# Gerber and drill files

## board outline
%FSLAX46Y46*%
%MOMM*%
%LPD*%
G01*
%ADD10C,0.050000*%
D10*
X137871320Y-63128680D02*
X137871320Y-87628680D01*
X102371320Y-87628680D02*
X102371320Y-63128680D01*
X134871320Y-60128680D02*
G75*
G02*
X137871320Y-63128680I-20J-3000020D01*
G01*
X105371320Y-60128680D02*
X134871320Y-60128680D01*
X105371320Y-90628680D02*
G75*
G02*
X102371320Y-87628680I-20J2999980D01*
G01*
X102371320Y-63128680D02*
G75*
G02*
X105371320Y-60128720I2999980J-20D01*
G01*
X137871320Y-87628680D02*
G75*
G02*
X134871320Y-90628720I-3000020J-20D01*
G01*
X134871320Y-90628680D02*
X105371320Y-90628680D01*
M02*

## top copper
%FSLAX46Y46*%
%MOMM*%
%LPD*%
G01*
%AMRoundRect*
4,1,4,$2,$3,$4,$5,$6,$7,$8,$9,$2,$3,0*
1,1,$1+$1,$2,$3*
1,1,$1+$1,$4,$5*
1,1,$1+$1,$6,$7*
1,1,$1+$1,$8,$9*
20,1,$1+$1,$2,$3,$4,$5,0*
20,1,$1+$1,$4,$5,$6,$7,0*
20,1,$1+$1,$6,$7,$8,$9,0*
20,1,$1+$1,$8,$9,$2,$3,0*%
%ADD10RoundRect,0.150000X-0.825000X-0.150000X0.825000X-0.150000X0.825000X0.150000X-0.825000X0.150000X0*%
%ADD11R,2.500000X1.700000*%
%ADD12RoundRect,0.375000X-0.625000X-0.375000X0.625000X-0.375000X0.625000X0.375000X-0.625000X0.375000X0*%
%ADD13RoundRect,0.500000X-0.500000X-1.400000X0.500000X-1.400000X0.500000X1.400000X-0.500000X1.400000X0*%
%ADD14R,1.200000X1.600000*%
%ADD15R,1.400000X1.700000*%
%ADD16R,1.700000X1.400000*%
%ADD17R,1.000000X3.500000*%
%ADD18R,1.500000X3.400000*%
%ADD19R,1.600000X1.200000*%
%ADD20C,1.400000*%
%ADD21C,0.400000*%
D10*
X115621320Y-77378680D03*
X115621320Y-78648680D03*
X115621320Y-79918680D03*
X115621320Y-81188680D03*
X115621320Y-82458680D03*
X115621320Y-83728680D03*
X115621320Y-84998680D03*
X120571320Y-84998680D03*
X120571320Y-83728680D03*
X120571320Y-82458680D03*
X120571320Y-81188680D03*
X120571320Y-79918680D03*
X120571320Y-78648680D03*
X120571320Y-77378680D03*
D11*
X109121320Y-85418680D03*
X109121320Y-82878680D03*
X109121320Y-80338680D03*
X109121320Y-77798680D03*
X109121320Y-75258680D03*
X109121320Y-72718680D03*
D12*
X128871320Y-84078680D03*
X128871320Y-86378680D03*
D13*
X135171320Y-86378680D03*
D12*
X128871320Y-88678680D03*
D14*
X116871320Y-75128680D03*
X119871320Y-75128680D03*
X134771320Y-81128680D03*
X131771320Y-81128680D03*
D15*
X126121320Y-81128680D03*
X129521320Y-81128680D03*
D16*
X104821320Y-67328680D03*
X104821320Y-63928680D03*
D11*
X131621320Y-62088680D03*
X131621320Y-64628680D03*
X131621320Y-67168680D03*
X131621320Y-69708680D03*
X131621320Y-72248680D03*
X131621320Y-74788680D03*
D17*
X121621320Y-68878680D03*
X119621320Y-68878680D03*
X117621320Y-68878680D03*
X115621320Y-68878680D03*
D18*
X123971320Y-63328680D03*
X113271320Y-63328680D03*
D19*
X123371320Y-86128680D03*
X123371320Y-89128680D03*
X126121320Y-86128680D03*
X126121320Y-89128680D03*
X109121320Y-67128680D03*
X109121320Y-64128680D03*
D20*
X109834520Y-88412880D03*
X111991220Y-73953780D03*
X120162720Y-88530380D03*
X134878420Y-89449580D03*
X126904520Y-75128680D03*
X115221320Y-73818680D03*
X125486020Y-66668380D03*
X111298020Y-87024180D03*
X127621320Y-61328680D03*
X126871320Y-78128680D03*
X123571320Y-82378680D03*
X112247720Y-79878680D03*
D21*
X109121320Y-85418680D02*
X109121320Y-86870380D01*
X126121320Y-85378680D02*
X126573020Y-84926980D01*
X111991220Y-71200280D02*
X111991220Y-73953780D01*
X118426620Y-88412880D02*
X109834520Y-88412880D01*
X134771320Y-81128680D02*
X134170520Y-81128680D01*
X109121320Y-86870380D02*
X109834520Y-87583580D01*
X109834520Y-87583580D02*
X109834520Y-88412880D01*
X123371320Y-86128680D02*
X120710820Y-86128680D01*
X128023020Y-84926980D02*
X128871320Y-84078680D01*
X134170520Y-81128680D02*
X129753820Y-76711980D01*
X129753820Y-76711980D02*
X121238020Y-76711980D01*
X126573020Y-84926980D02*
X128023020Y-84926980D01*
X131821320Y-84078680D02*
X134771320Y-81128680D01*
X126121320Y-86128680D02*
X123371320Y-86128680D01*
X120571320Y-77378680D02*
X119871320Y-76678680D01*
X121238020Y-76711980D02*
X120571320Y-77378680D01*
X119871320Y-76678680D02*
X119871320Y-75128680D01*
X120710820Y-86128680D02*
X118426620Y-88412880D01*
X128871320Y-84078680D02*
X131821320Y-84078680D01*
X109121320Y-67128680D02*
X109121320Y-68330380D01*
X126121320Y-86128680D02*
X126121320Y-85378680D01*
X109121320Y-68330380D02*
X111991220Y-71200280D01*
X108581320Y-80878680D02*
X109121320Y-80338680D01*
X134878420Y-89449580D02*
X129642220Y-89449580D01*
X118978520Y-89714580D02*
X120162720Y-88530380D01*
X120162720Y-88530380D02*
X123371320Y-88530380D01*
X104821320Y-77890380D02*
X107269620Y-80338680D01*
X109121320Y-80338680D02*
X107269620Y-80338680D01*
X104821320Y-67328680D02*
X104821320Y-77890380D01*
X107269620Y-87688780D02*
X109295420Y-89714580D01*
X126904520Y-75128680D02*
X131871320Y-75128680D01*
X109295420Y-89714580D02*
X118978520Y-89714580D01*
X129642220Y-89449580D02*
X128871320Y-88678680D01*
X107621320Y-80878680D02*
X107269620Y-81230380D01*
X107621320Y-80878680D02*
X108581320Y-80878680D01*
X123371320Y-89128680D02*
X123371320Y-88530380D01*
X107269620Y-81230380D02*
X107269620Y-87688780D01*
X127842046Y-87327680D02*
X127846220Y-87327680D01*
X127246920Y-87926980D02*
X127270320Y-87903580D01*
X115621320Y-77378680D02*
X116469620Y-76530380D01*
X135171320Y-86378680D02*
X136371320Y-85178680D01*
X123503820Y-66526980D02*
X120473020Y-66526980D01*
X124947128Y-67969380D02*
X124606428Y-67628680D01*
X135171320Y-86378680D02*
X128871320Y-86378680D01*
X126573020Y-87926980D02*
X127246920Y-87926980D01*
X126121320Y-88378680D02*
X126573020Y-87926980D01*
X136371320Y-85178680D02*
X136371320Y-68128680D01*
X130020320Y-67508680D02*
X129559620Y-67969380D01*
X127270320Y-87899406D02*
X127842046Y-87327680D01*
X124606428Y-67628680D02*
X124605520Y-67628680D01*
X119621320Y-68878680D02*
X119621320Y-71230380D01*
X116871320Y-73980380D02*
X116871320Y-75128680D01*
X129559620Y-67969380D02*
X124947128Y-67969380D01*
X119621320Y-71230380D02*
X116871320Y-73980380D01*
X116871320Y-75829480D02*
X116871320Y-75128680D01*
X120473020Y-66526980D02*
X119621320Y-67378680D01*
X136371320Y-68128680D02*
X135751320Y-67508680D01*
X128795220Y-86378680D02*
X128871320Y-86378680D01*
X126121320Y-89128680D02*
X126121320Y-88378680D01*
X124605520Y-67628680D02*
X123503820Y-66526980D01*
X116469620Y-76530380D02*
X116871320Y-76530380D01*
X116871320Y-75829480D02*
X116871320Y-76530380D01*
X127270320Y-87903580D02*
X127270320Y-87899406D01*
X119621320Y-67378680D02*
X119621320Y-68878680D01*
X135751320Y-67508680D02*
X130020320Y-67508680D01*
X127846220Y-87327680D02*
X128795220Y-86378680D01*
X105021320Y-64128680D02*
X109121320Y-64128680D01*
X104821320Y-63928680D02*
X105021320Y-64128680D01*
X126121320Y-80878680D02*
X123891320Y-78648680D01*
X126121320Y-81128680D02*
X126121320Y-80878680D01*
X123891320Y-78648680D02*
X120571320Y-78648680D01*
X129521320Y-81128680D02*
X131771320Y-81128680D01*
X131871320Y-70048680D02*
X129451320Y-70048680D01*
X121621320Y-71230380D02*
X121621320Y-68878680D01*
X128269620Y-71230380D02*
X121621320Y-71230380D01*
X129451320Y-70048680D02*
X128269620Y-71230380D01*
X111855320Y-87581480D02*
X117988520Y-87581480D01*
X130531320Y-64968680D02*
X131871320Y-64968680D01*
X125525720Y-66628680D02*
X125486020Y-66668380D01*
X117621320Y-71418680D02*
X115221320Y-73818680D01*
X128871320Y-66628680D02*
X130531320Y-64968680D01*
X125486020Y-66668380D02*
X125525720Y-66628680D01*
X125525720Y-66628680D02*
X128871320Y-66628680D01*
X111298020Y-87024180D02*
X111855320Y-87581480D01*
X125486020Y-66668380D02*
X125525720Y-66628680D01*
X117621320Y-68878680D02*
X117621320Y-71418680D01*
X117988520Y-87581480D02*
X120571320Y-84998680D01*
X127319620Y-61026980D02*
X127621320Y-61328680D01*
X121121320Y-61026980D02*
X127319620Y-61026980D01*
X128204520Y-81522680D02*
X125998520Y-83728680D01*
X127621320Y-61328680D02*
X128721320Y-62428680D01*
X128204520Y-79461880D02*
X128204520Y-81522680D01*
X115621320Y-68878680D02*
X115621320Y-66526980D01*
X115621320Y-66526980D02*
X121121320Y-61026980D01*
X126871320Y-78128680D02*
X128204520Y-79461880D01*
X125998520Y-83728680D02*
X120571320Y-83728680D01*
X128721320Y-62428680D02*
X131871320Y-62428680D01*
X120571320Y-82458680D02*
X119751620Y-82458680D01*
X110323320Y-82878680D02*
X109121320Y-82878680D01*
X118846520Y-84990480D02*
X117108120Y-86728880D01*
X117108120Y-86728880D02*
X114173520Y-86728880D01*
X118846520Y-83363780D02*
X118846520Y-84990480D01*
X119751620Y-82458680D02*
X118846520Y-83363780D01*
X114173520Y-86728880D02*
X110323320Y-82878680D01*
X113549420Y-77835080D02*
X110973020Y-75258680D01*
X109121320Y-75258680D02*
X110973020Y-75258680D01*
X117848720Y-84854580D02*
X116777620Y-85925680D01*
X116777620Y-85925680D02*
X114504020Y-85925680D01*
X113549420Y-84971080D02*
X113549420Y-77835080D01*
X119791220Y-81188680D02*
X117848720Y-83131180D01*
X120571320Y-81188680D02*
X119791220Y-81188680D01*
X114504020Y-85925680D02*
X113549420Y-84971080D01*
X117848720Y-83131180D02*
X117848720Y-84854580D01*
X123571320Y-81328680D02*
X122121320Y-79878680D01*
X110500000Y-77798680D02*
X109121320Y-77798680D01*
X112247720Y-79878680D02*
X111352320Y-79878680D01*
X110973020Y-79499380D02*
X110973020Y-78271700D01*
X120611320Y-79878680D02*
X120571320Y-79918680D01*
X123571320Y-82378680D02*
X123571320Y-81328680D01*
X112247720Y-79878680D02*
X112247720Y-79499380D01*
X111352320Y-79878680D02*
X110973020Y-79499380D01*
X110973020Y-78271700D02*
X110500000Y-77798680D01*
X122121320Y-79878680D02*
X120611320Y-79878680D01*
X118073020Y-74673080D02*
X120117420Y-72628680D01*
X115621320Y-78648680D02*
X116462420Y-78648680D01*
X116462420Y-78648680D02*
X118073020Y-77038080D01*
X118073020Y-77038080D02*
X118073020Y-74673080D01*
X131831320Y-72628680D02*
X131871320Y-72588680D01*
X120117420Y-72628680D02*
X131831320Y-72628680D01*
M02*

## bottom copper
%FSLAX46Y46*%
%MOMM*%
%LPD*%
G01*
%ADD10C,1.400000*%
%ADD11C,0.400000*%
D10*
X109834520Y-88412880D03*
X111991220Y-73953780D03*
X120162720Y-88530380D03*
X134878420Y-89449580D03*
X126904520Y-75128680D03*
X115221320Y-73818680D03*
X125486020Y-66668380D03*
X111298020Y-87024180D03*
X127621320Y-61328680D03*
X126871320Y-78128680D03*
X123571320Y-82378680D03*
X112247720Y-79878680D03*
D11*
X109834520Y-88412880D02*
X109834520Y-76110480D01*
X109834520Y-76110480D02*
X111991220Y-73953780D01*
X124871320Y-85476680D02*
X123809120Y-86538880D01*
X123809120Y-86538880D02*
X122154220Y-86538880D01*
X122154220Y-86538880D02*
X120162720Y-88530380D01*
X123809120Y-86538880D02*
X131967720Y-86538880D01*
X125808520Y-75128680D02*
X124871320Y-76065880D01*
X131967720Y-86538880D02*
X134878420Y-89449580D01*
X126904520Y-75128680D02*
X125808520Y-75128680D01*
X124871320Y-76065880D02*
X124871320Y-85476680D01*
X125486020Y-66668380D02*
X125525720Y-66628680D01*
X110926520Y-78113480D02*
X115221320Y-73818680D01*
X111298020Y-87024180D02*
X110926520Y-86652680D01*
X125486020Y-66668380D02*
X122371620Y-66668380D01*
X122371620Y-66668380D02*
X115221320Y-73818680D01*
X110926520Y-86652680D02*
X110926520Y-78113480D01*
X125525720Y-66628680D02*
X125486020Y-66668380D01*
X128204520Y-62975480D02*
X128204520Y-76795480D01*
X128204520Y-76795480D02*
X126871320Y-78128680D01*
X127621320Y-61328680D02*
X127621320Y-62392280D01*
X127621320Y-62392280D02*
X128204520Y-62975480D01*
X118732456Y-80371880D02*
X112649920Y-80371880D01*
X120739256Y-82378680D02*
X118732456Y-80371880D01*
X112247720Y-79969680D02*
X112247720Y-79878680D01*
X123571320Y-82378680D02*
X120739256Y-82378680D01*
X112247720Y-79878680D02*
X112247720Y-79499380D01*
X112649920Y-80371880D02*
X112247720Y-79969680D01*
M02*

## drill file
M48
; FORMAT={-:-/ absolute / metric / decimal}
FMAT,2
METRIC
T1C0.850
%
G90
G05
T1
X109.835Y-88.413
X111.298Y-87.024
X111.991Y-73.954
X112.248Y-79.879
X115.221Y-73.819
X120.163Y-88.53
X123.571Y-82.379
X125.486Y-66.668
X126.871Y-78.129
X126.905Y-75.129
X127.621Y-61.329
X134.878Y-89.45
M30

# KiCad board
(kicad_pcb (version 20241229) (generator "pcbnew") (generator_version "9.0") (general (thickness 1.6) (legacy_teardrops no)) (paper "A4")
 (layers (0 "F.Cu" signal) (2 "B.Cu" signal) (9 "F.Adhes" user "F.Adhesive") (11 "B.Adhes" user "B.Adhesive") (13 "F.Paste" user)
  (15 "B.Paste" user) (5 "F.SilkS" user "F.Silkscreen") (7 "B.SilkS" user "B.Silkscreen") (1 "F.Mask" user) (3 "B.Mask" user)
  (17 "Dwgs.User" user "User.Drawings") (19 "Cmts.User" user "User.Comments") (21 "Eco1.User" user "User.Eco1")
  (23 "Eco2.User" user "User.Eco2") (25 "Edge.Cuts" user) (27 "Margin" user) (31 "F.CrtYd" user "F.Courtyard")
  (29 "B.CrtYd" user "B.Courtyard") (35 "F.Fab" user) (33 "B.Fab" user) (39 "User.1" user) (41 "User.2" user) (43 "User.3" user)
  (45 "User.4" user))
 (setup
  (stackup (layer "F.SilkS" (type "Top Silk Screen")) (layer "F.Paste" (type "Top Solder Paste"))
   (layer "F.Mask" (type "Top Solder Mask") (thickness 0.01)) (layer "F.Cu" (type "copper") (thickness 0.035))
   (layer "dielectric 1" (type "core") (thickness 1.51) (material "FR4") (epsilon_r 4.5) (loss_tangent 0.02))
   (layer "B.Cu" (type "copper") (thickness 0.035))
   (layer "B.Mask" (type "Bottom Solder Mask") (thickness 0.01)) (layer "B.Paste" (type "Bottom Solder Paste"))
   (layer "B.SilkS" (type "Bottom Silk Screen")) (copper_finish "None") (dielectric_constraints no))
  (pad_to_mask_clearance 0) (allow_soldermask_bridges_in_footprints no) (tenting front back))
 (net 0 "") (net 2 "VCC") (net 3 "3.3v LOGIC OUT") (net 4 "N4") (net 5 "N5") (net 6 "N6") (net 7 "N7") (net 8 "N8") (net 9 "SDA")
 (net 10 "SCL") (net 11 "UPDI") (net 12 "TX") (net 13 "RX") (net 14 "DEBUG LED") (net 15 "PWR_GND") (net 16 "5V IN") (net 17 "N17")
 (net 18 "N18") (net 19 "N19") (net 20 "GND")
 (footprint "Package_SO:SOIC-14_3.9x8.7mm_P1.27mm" (layer "F.Cu") (at 118.09632 81.18868)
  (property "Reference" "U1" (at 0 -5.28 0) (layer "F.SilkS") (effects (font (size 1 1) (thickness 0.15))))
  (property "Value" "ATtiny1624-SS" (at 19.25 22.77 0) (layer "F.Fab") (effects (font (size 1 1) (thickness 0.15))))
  (pad "1" smd roundrect (at -2.475 -3.81) (size 1.95 0.6) (layers "F.Cu" "F.Mask" "F.Paste") (roundrect_rratio 0.25) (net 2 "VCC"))
  (pad "2" smd roundrect (at -2.475 -2.54) (size 1.95 0.6) (layers "F.Cu" "F.Mask" "F.Paste") (roundrect_rratio 0.25)
   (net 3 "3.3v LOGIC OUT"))
  (pad "3" smd roundrect (at -2.475 -1.27) (size 1.95 0.6) (layers "F.Cu" "F.Mask" "F.Paste") (roundrect_rratio 0.25) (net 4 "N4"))
  (pad "4" smd roundrect (at -2.475 0) (size 1.95 0.6) (layers "F.Cu" "F.Mask" "F.Paste") (roundrect_rratio 0.25) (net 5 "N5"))
  (pad "5" smd roundrect (at -2.475 1.27) (size 1.95 0.6) (layers "F.Cu" "F.Mask" "F.Paste") (roundrect_rratio 0.25) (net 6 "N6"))
  (pad "6" smd roundrect (at -2.475 2.54) (size 1.95 0.6) (layers "F.Cu" "F.Mask" "F.Paste") (roundrect_rratio 0.25) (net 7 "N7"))
  (pad "7" smd roundrect (at -2.475 3.81) (size 1.95 0.6) (layers "F.Cu" "F.Mask" "F.Paste") (roundrect_rratio 0.25) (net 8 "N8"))
  (pad "8" smd roundrect (at 2.475 3.81) (size 1.95 0.6) (layers "F.Cu" "F.Mask" "F.Paste") (roundrect_rratio 0.25) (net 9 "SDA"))
  (pad "9" smd roundrect (at 2.475 2.54) (size 1.95 0.6) (layers "F.Cu" "F.Mask" "F.Paste") (roundrect_rratio 0.25) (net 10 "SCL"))
  (pad "10" smd roundrect (at 2.475 1.27) (size 1.95 0.6) (layers "F.Cu" "F.Mask" "F.Paste") (roundrect_rratio 0.25) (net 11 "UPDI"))
  (pad "11" smd roundrect (at 2.475 0) (size 1.95 0.6) (layers "F.Cu" "F.Mask" "F.Paste") (roundrect_rratio 0.25) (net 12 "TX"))
  (pad "12" smd roundrect (at 2.475 -1.27) (size 1.95 0.6) (layers "F.Cu" "F.Mask" "F.Paste") (roundrect_rratio 0.25) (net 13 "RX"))
  (pad "13" smd roundrect (at 2.475 -2.54) (size 1.95 0.6) (layers "F.Cu" "F.Mask" "F.Paste") (roundrect_rratio 0.25) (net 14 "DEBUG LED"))
  (pad "14" smd roundrect (at 2.475 -3.81) (size 1.95 0.6) (layers "F.Cu" "F.Mask" "F.Paste") (roundrect_rratio 0.25) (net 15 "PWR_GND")))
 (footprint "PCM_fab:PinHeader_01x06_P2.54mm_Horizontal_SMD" (layer "F.Cu") (at 109.12132 85.41868 180)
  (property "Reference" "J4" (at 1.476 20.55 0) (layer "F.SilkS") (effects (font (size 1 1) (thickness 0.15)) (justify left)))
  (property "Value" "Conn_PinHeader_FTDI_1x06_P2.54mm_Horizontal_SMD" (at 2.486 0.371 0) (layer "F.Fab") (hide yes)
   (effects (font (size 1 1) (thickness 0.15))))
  (pad "1" smd rect (at 0 0 180) (size 2.5 1.7) (layers "F.Cu" "F.Mask" "F.Paste") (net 15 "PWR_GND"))
  (pad "2" smd rect (at 0 2.54 180) (size 2.5 1.7) (layers "F.Cu" "F.Mask" "F.Paste") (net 11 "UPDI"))
  (pad "3" smd rect (at 0 5.08 180) (size 2.5 1.7) (layers "F.Cu" "F.Mask" "F.Paste") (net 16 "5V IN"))
  (pad "4" smd rect (at 0 7.62 180) (size 2.5 1.7) (layers "F.Cu" "F.Mask" "F.Paste") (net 13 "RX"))
  (pad "5" smd rect (at 0 10.16 180) (size 2.5 1.7) (layers "F.Cu" "F.Mask" "F.Paste") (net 12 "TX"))
  (pad "6" smd rect (at 0 12.7 180) (size 2.5 1.7) (layers "F.Cu" "F.Mask" "F.Paste") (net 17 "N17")))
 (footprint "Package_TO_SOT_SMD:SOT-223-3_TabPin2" (layer "F.Cu") (at 132.02132 86.37868)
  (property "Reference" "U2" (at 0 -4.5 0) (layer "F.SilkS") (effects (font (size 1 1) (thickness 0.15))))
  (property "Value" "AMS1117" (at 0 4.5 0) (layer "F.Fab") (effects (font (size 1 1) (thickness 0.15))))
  (pad "1" smd roundrect (at -3.15 -2.3) (size 2 1.5) (layers "F.Cu" "F.Mask" "F.Paste") (roundrect_rratio 0.25) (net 15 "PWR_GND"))
  (pad "2" smd roundrect (at -3.15 0) (size 2 1.5) (layers "F.Cu" "F.Mask" "F.Paste") (roundrect_rratio 0.25) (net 2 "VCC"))
  (pad "2" smd roundrect (at 3.15 0) (size 2 3.8) (layers "F.Cu" "F.Mask" "F.Paste") (roundrect_rratio 0.25) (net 2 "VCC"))
  (pad "3" smd roundrect (at -3.15 2.3) (size 2 1.5) (layers "F.Cu" "F.Mask" "F.Paste") (roundrect_rratio 0.25) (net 16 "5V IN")))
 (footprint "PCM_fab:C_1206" (layer "F.Cu") (at 118.37132 75.12868)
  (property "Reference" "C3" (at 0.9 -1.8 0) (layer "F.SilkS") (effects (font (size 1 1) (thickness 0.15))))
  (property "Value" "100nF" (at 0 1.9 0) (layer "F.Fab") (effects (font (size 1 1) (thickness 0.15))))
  (pad "1" smd rect (at -1.5 0) (size 1.2 1.6) (layers "F.Cu" "F.Mask" "F.Paste") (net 2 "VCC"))
  (pad "2" smd rect (at 1.5 0) (size 1.2 1.6) (layers "F.Cu" "F.Mask" "F.Paste") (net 15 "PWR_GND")))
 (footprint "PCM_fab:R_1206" (layer "F.Cu") (at 133.27132 81.12868 180)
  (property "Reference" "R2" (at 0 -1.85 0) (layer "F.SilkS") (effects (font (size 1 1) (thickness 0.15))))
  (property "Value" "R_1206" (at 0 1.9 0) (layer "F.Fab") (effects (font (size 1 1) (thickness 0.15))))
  (pad "1" smd rect (at -1.5 0 180) (size 1.2 1.6) (layers "F.Cu" "F.Mask" "F.Paste") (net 15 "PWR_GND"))
  (pad "2" smd rect (at 1.5 0 180) (size 1.2 1.6) (layers "F.Cu" "F.Mask" "F.Paste") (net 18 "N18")))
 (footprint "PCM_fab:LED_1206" (layer "F.Cu") (at 127.82132 81.12868)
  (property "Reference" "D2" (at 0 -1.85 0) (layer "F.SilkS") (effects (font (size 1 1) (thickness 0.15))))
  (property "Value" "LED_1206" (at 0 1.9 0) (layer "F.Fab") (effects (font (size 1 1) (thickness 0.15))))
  (pad "1" smd rect (at -1.7 0) (size 1.4 1.7) (layers "F.Cu" "F.Mask" "F.Paste") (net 14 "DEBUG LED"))
  (pad "2" smd rect (at 1.7 0) (size 1.4 1.7) (layers "F.Cu" "F.Mask" "F.Paste") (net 18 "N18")))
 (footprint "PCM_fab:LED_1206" (layer "F.Cu") (at 104.82132 65.62868 90)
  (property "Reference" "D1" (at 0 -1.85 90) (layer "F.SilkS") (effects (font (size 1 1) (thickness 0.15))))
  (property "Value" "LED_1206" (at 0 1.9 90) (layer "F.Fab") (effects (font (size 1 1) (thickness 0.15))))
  (pad "1" smd rect (at -1.7 0 90) (size 1.4 1.7) (layers "F.Cu" "F.Mask" "F.Paste") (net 16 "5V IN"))
  (pad "2" smd rect (at 1.7 0 90) (size 1.4 1.7) (layers "F.Cu" "F.Mask" "F.Paste") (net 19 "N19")))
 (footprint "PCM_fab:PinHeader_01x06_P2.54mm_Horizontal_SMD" (layer "F.Cu") (at 131.62132 62.08868)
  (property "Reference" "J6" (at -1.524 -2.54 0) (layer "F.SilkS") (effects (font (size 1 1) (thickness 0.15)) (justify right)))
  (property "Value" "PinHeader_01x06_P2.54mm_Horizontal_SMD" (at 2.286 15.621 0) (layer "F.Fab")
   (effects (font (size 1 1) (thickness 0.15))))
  (pad "1" smd rect (at 0 0) (size 2.5 1.7) (layers "F.Cu" "F.Mask" "F.Paste") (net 10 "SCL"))
  (pad "2" smd rect (at 0 2.54) (size 2.5 1.7) (layers "F.Cu" "F.Mask" "F.Paste") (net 9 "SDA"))
  (pad "3" smd rect (at 0 5.08) (size 2.5 1.7) (layers "F.Cu" "F.Mask" "F.Paste") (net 2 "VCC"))
  (pad "4" smd rect (at 0 7.62) (size 2.5 1.7) (layers "F.Cu" "F.Mask" "F.Paste") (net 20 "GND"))
  (pad "5" smd rect (at 0 10.16) (size 2.5 1.7) (layers "F.Cu" "F.Mask" "F.Paste") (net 3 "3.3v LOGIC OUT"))
  (pad "6" smd rect (at 0 12.7) (size 2.5 1.7) (layers "F.Cu" "F.Mask" "F.Paste") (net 16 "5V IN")))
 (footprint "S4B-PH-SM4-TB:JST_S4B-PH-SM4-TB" (layer "F.Cu") (at 118.62132 66.12868 180)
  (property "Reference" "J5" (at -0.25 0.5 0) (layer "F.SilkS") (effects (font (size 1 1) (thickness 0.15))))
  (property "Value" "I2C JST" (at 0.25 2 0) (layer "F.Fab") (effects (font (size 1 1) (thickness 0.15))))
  (pad "1" smd rect (at -3 -2.75 180) (size 1 3.5) (layers "F.Cu" "F.Mask" "F.Paste") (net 20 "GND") (solder_mask_margin 0.102))
  (pad "2" smd rect (at -1 -2.75 180) (size 1 3.5) (layers "F.Cu" "F.Mask" "F.Paste") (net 2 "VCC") (solder_mask_margin 0.102))
  (pad "3" smd rect (at 1 -2.75 180) (size 1 3.5) (layers "F.Cu" "F.Mask" "F.Paste") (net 9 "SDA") (solder_mask_margin 0.102))
  (pad "4" smd rect (at 3 -2.75 180) (size 1 3.5) (layers "F.Cu" "F.Mask" "F.Paste") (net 10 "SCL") (solder_mask_margin 0.102))
  (pad "SH1" smd rect (at -5.35 2.8 180) (size 1.5 3.4) (layers "F.Cu" "F.Mask" "F.Paste") (solder_mask_margin 0.102))
  (pad "SH2" smd rect (at 5.35 2.8 180) (size 1.5 3.4) (layers "F.Cu" "F.Mask" "F.Paste") (solder_mask_margin 0.102)))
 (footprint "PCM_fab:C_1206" (layer "F.Cu") (at 123.37132 87.62868 -90)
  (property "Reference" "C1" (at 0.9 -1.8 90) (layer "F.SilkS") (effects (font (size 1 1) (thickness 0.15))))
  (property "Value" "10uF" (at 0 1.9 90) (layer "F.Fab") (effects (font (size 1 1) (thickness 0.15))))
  (pad "1" smd rect (at -1.5 0 270) (size 1.2 1.6) (layers "F.Cu" "F.Mask" "F.Paste") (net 15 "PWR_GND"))
  (pad "2" smd rect (at 1.5 0 270) (size 1.2 1.6) (layers "F.Cu" "F.Mask" "F.Paste") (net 16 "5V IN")))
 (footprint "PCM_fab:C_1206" (layer "F.Cu") (at 126.12132 87.62868 -90)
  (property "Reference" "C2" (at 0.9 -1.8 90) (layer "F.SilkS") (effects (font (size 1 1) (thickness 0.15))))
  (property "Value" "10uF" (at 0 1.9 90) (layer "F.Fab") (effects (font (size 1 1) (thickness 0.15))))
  (pad "1" smd rect (at -1.5 0 270) (size 1.2 1.6) (layers "F.Cu" "F.Mask" "F.Paste") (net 15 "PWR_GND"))
  (pad "2" smd rect (at 1.5 0 270) (size 1.2 1.6) (layers "F.Cu" "F.Mask" "F.Paste") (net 2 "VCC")))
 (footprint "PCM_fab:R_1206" (layer "F.Cu") (at 109.12132 65.62868 90)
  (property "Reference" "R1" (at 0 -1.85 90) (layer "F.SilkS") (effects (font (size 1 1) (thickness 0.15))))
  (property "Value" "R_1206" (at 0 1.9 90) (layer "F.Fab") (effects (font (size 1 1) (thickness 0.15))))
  (pad "1" smd rect (at -1.5 0 90) (size 1.2 1.6) (layers "F.Cu" "F.Mask" "F.Paste") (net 15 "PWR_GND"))
  (pad "2" smd rect (at 1.5 0 90) (size 1.2 1.6) (layers "F.Cu" "F.Mask" "F.Paste") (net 19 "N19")))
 (gr_line (start 137.87132 63.12868) (end 137.87132 87.62868) (stroke (width 0.05) (type default)) (layer "Edge.Cuts"))
 (gr_line (start 102.37132 87.62868) (end 102.37132 63.12868) (stroke (width 0.05) (type default)) (layer "Edge.Cuts"))
 (gr_arc (start 134.87132 60.12868) (mid 136.99264 61.00736) (end 137.87132 63.12868) (stroke (width 0.05) (type default))
  (layer "Edge.Cuts"))
 (gr_line (start 105.37132 60.12868) (end 134.87132 60.12868) (stroke (width 0.05) (type default)) (layer "Edge.Cuts"))
 (gr_arc (start 105.37132 90.62868) (mid 103.25 89.75) (end 102.37132 87.62868) (stroke (width 0.05) (type default)) (layer "Edge.Cuts"))
 (gr_arc (start 102.37132 63.12868) (mid 103.25 61.00736) (end 105.37132 60.12868) (stroke (width 0.05) (type default)) (layer "Edge.Cuts"))
 (gr_arc (start 137.87132 87.62868) (mid 136.99264 89.75) (end 134.87132 90.62868) (stroke (width 0.05) (type default)) (layer "Edge.Cuts"))
 (gr_line (start 134.87132 90.62868) (end 105.37132 90.62868) (stroke (width 0.05) (type default)) (layer "Edge.Cuts"))
 (segment (start 109.12132 85.41868) (end 109.12132 86.87038) (width 0.4) (layer "F.Cu") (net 15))
 (segment (start 126.12132 85.37868) (end 126.57302 84.92698) (width 0.4) (layer "F.Cu") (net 15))
 (segment (start 111.99122 71.20028) (end 111.99122 73.95378) (width 0.4) (layer "F.Cu") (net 15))
 (segment (start 118.42662 88.41288) (end 109.83452 88.41288) (width 0.4) (layer "F.Cu") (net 15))
 (segment (start 134.77132 81.12868) (end 134.17052 81.12868) (width 0.4) (layer "F.Cu") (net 15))
 (segment (start 109.12132 86.87038) (end 109.83452 87.58358) (width 0.4) (layer "F.Cu") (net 15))
 (segment (start 109.83452 87.58358) (end 109.83452 88.41288) (width 0.4) (layer "F.Cu") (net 15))
 (segment (start 123.37132 86.12868) (end 120.71082 86.12868) (width 0.4) (layer "F.Cu") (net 15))
 (segment (start 128.02302 84.92698) (end 128.87132 84.07868) (width 0.4) (layer "F.Cu") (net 15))
 (segment (start 134.17052 81.12868) (end 129.75382 76.71198) (width 0.4) (layer "F.Cu") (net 15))
 (segment (start 129.75382 76.71198) (end 121.23802 76.71198) (width 0.4) (layer "F.Cu") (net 15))
 (segment (start 126.57302 84.92698) (end 128.02302 84.92698) (width 0.4) (layer "F.Cu") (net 15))
 (segment (start 131.82132 84.07868) (end 134.77132 81.12868) (width 0.4) (layer "F.Cu") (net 15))
 (segment (start 126.12132 86.12868) (end 123.37132 86.12868) (width 0.4) (layer "F.Cu") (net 15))
 (segment (start 120.57132 77.37868) (end 119.87132 76.67868) (width 0.4) (layer "F.Cu") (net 15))
 (segment (start 121.23802 76.71198) (end 120.57132 77.37868) (width 0.4) (layer "F.Cu") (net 15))
 (segment (start 119.87132 76.67868) (end 119.87132 75.12868) (width 0.4) (layer "F.Cu") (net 15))
 (segment (start 120.71082 86.12868) (end 118.42662 88.41288) (width 0.4) (layer "F.Cu") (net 15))
 (segment (start 128.87132 84.07868) (end 131.82132 84.07868) (width 0.4) (layer "F.Cu") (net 15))
 (segment (start 109.12132 67.12868) (end 109.12132 68.33038) (width 0.4) (layer "F.Cu") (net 15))
 (segment (start 126.12132 86.12868) (end 126.12132 85.37868) (width 0.4) (layer "F.Cu") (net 15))
 (segment (start 109.12132 68.33038) (end 111.99122 71.20028) (width 0.4) (layer "F.Cu") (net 15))
 (via (at 109.83452 88.41288) (size 1.4) (drill 0.85) (layers "F.Cu" "B.Cu") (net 15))
 (via (at 111.99122 73.95378) (size 1.4) (drill 0.85) (layers "F.Cu" "B.Cu") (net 15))
 (segment (start 109.83452 88.41288) (end 109.83452 76.11048) (width 0.4) (layer "B.Cu") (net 15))
 (segment (start 109.83452 76.11048) (end 111.99122 73.95378) (width 0.4) (layer "B.Cu") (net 15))
 (segment (start 108.58132 80.87868) (end 109.12132 80.33868) (width 0.4) (layer "F.Cu") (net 16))
 (segment (start 134.87842 89.44958) (end 129.64222 89.44958) (width 0.4) (layer "F.Cu") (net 16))
 (segment (start 118.97852 89.71458) (end 120.16272 88.53038) (width 0.4) (layer "F.Cu") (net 16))
 (segment (start 120.16272 88.53038) (end 123.37132 88.53038) (width 0.4) (layer "F.Cu") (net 16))
 (segment (start 104.82132 77.89038) (end 107.26962 80.33868) (width 0.4) (layer "F.Cu") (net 16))
 (segment (start 109.12132 80.33868) (end 107.26962 80.33868) (width 0.4) (layer "F.Cu") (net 16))
 (segment (start 104.82132 67.32868) (end 104.82132 77.89038) (width 0.4) (layer "F.Cu") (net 16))
 (segment (start 107.26962 87.68878) (end 109.29542 89.71458) (width 0.4) (layer "F.Cu") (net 16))
 (segment (start 126.90452 75.12868) (end 131.87132 75.12868) (width 0.4) (layer "F.Cu") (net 16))
 (segment (start 109.29542 89.71458) (end 118.97852 89.71458) (width 0.4) (layer "F.Cu") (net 16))
 (segment (start 129.64222 89.44958) (end 128.87132 88.67868) (width 0.4) (layer "F.Cu") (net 16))
 (segment (start 107.62132 80.87868) (end 107.26962 81.23038) (width 0.4) (layer "F.Cu") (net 16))
 (segment (start 107.62132 80.87868) (end 108.58132 80.87868) (width 0.4) (layer "F.Cu") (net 16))
 (segment (start 123.37132 89.12868) (end 123.37132 88.53038) (width 0.4) (layer "F.Cu") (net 16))
 (segment (start 107.26962 81.23038) (end 107.26962 87.68878) (width 0.4) (layer "F.Cu") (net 16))
 (via (at 120.16272 88.53038) (size 1.4) (drill 0.85) (layers "F.Cu" "B.Cu") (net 16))
 (via (at 134.87842 89.44958) (size 1.4) (drill 0.85) (layers "F.Cu" "B.Cu") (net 16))
 (via (at 126.90452 75.12868) (size 1.4) (drill 0.85) (layers "F.Cu" "B.Cu") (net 16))
 (segment (start 124.87132 85.47668) (end 123.80912 86.53888) (width 0.4) (layer "B.Cu") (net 16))
 (segment (start 123.80912 86.53888) (end 122.15422 86.53888) (width 0.4) (layer "B.Cu") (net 16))
 (segment (start 122.15422 86.53888) (end 120.16272 88.53038) (width 0.4) (layer "B.Cu") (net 16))
 (segment (start 123.80912 86.53888) (end 131.96772 86.53888) (width 0.4) (layer "B.Cu") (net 16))
 (segment (start 125.80852 75.12868) (end 124.87132 76.06588) (width 0.4) (layer "B.Cu") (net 16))
 (segment (start 131.96772 86.53888) (end 134.87842 89.44958) (width 0.4) (layer "B.Cu") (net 16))
 (segment (start 126.90452 75.12868) (end 125.80852 75.12868) (width 0.4) (layer "B.Cu") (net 16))
 (segment (start 124.87132 76.06588) (end 124.87132 85.47668) (width 0.4) (layer "B.Cu") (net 16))
 (segment (start 127.842046 87.32768) (end 127.84622 87.32768) (width 0.4) (layer "F.Cu") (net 2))
 (segment (start 127.24692 87.92698) (end 127.27032 87.90358) (width 0.4) (layer "F.Cu") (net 2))
 (segment (start 115.62132 77.37868) (end 116.46962 76.53038) (width 0.4) (layer "F.Cu") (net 2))
 (segment (start 135.17132 86.37868) (end 136.37132 85.17868) (width 0.4) (layer "F.Cu") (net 2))
 (segment (start 123.50382 66.52698) (end 120.47302 66.52698) (width 0.4) (layer "F.Cu") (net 2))
 (segment (start 124.947128 67.96938) (end 124.606428 67.62868) (width 0.4) (layer "F.Cu") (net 2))
 (segment (start 135.17132 86.37868) (end 128.87132 86.37868) (width 0.4) (layer "F.Cu") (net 2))
 (segment (start 126.57302 87.92698) (end 127.24692 87.92698) (width 0.4) (layer "F.Cu") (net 2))
 (segment (start 126.12132 88.37868) (end 126.57302 87.92698) (width 0.4) (layer "F.Cu") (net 2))
 (segment (start 136.37132 85.17868) (end 136.37132 68.12868) (width 0.4) (layer "F.Cu") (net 2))
 (segment (start 130.02032 67.50868) (end 129.55962 67.96938) (width 0.4) (layer "F.Cu") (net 2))
 (segment (start 127.27032 87.899406) (end 127.842046 87.32768) (width 0.4) (layer "F.Cu") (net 2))
 (segment (start 124.606428 67.62868) (end 124.60552 67.62868) (width 0.4) (layer "F.Cu") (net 2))
 (segment (start 119.62132 68.87868) (end 119.62132 71.23038) (width 0.4) (layer "F.Cu") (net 2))
 (segment (start 116.87132 73.98038) (end 116.87132 75.12868) (width 0.4) (layer "F.Cu") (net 2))
 (segment (start 129.55962 67.96938) (end 124.947128 67.96938) (width 0.4) (layer "F.Cu") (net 2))
 (segment (start 119.62132 71.23038) (end 116.87132 73.98038) (width 0.4) (layer "F.Cu") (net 2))
 (segment (start 116.87132 75.82948) (end 116.87132 75.12868) (width 0.4) (layer "F.Cu") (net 2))
 (segment (start 120.47302 66.52698) (end 119.62132 67.37868) (width 0.4) (layer "F.Cu") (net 2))
 (segment (start 136.37132 68.12868) (end 135.75132 67.50868) (width 0.4) (layer "F.Cu") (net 2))
 (segment (start 128.79522 86.37868) (end 128.87132 86.37868) (width 0.4) (layer "F.Cu") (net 2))
 (segment (start 126.12132 89.12868) (end 126.12132 88.37868) (width 0.4) (layer "F.Cu") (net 2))
 (segment (start 124.60552 67.62868) (end 123.50382 66.52698) (width 0.4) (layer "F.Cu") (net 2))
 (segment (start 116.46962 76.53038) (end 116.87132 76.53038) (width 0.4) (layer "F.Cu") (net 2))
 (segment (start 116.87132 75.82948) (end 116.87132 76.53038) (width 0.4) (layer "F.Cu") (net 2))
 (segment (start 127.27032 87.90358) (end 127.27032 87.899406) (width 0.4) (layer "F.Cu") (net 2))
 (segment (start 119.62132 67.37868) (end 119.62132 68.87868) (width 0.4) (layer "F.Cu") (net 2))
 (segment (start 135.75132 67.50868) (end 130.02032 67.50868) (width 0.4) (layer "F.Cu") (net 2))
 (segment (start 127.84622 87.32768) (end 128.79522 86.37868) (width 0.4) (layer "F.Cu") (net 2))
 (segment (start 105.02132 64.12868) (end 109.12132 64.12868) (width 0.4) (layer "F.Cu") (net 19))
 (segment (start 104.82132 63.92868) (end 105.02132 64.12868) (width 0.4) (layer "F.Cu") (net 19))
 (segment (start 126.12132 80.87868) (end 123.89132 78.64868) (width 0.4) (layer "F.Cu") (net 14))
 (segment (start 126.12132 81.12868) (end 126.12132 80.87868) (width 0.4) (layer "F.Cu") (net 14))
 (segment (start 123.89132 78.64868) (end 120.57132 78.64868) (width 0.4) (layer "F.Cu") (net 14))
 (segment (start 129.52132 81.12868) (end 131.77132 81.12868) (width 0.4) (layer "F.Cu") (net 18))
 (segment (start 131.87132 70.04868) (end 129.45132 70.04868) (width 0.4) (layer "F.Cu") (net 20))
 (segment (start 121.62132 71.23038) (end 121.62132 68.87868) (width 0.4) (layer "F.Cu") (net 20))
 (segment (start 128.26962 71.23038) (end 121.62132 71.23038) (width 0.4) (layer "F.Cu") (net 20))
 (segment (start 129.45132 70.04868) (end 128.26962 71.23038) (width 0.4) (layer "F.Cu") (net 20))
 (segment (start 111.85532 87.58148) (end 117.98852 87.58148) (width 0.4) (layer "F.Cu") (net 9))
 (segment (start 130.53132 64.96868) (end 131.87132 64.96868) (width 0.4) (layer "F.Cu") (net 9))
 (segment (start 125.52572 66.62868) (end 125.48602 66.66838) (width 0.4) (layer "F.Cu") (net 9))
 (segment (start 117.62132 71.41868) (end 115.22132 73.81868) (width 0.4) (layer "F.Cu") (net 9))
 (segment (start 128.87132 66.62868) (end 130.53132 64.96868) (width 0.4) (layer "F.Cu") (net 9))
 (segment (start 125.48602 66.66838) (end 125.52572 66.62868) (width 0.4) (layer "F.Cu") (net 9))
 (segment (start 125.52572 66.62868) (end 128.87132 66.62868) (width 0.4) (layer "F.Cu") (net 9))
 (segment (start 111.29802 87.02418) (end 111.85532 87.58148) (width 0.4) (layer "F.Cu") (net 9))
 (segment (start 125.48602 66.66838) (end 125.52572 66.62868) (width 0.4) (layer "F.Cu") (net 9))
 (segment (start 117.62132 68.87868) (end 117.62132 71.41868) (width 0.4) (layer "F.Cu") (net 9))
 (segment (start 117.98852 87.58148) (end 120.57132 84.99868) (width 0.4) (layer "F.Cu") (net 9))
 (via (at 115.22132 73.81868) (size 1.4) (drill 0.85) (layers "F.Cu" "B.Cu") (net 9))
 (via (at 125.48602 66.66838) (size 1.4) (drill 0.85) (layers "F.Cu" "B.Cu") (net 9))
 (via (at 111.29802 87.02418) (size 1.4) (drill 0.85) (layers "F.Cu" "B.Cu") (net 9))
 (segment (start 125.48602 66.66838) (end 125.52572 66.62868) (width 0.4) (layer "B.Cu") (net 9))
 (segment (start 110.92652 78.11348) (end 115.22132 73.81868) (width 0.4) (layer "B.Cu") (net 9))
 (segment (start 111.29802 87.02418) (end 110.92652 86.65268) (width 0.4) (layer "B.Cu") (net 9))
 (segment (start 125.48602 66.66838) (end 122.37162 66.66838) (width 0.4) (layer "B.Cu") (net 9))
 (segment (start 122.37162 66.66838) (end 115.22132 73.81868) (width 0.4) (layer "B.Cu") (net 9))
 (segment (start 110.92652 86.65268) (end 110.92652 78.11348) (width 0.4) (layer "B.Cu") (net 9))
 (segment (start 125.52572 66.62868) (end 125.48602 66.66838) (width 0.4) (layer "B.Cu") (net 9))
 (segment (start 127.31962 61.02698) (end 127.62132 61.32868) (width 0.4) (layer "F.Cu") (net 10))
 (segment (start 121.12132 61.02698) (end 127.31962 61.02698) (width 0.4) (layer "F.Cu") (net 10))
 (segment (start 128.20452 81.52268) (end 125.99852 83.72868) (width 0.4) (layer "F.Cu") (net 10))
 (segment (start 127.62132 61.32868) (end 128.72132 62.42868) (width 0.4) (layer "F.Cu") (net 10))
 (segment (start 128.20452 79.46188) (end 128.20452 81.52268) (width 0.4) (layer "F.Cu") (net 10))
 (segment (start 115.62132 68.87868) (end 115.62132 66.52698) (width 0.4) (layer "F.Cu") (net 10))
 (segment (start 115.62132 66.52698) (end 121.12132 61.02698) (width 0.4) (layer "F.Cu") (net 10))
 (segment (start 126.87132 78.12868) (end 128.20452 79.46188) (width 0.4) (layer "F.Cu") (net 10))
 (segment (start 125.99852 83.72868) (end 120.57132 83.72868) (width 0.4) (layer "F.Cu") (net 10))
 (segment (start 128.72132 62.42868) (end 131.87132 62.42868) (width 0.4) (layer "F.Cu") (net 10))
 (via (at 127.62132 61.32868) (size 1.4) (drill 0.85) (layers "F.Cu" "B.Cu") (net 10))
 (via (at 126.87132 78.12868) (size 1.4) (drill 0.85) (layers "F.Cu" "B.Cu") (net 10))
 (segment (start 128.20452 62.97548) (end 128.20452 76.79548) (width 0.4) (layer "B.Cu") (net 10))
 (segment (start 128.20452 76.79548) (end 126.87132 78.12868) (width 0.4) (layer "B.Cu") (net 10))
 (segment (start 127.62132 61.32868) (end 127.62132 62.39228) (width 0.4) (layer "B.Cu") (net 10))
 (segment (start 127.62132 62.39228) (end 128.20452 62.97548) (width 0.4) (layer "B.Cu") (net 10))
 (segment (start 120.57132 82.45868) (end 119.75162 82.45868) (width 0.4) (layer "F.Cu") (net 11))
 (segment (start 110.32332 82.87868) (end 109.12132 82.87868) (width 0.4) (layer "F.Cu") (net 11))
 (segment (start 118.84652 84.99048) (end 117.10812 86.72888) (width 0.4) (layer "F.Cu") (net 11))
 (segment (start 117.10812 86.72888) (end 114.17352 86.72888) (width 0.4) (layer "F.Cu") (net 11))
 (segment (start 118.84652 83.36378) (end 118.84652 84.99048) (width 0.4) (layer "F.Cu") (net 11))
 (segment (start 119.75162 82.45868) (end 118.84652 83.36378) (width 0.4) (layer "F.Cu") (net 11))
 (segment (start 114.17352 86.72888) (end 110.32332 82.87868) (width 0.4) (layer "F.Cu") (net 11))
 (segment (start 113.54942 77.83508) (end 110.97302 75.25868) (width 0.4) (layer "F.Cu") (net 12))
 (segment (start 109.12132 75.25868) (end 110.97302 75.25868) (width 0.4) (layer "F.Cu") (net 12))
 (segment (start 117.84872 84.85458) (end 116.77762 85.92568) (width 0.4) (layer "F.Cu") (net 12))
 (segment (start 116.77762 85.92568) (end 114.50402 85.92568) (width 0.4) (layer "F.Cu") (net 12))
 (segment (start 113.54942 84.97108) (end 113.54942 77.83508) (width 0.4) (layer "F.Cu") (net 12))
 (segment (start 119.79122 81.18868) (end 117.84872 83.13118) (width 0.4) (layer "F.Cu") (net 12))
 (segment (start 120.57132 81.18868) (end 119.79122 81.18868) (width 0.4) (layer "F.Cu") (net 12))
 (segment (start 114.50402 85.92568) (end 113.54942 84.97108) (width 0.4) (layer "F.Cu") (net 12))
 (segment (start 117.84872 83.13118) (end 117.84872 84.85458) (width 0.4) (layer "F.Cu") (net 12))
 (segment (start 123.57132 81.32868) (end 122.12132 79.87868) (width 0.4) (layer "F.Cu") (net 13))
 (segment (start 110.5 77.79868) (end 109.12132 77.79868) (width 0.4) (layer "F.Cu") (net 13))
 (segment (start 112.24772 79.87868) (end 111.35232 79.87868) (width 0.4) (layer "F.Cu") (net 13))
 (segment (start 110.97302 79.49938) (end 110.97302 78.2717) (width 0.4) (layer "F.Cu") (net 13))
 (segment (start 120.61132 79.87868) (end 120.57132 79.91868) (width 0.4) (layer "F.Cu") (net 13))
 (segment (start 123.57132 82.37868) (end 123.57132 81.32868) (width 0.4) (layer "F.Cu") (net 13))
 (segment (start 112.24772 79.87868) (end 112.24772 79.49938) (width 0.4) (layer "F.Cu") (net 13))
 (segment (start 111.35232 79.87868) (end 110.97302 79.49938) (width 0.4) (layer "F.Cu") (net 13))
 (segment (start 110.97302 78.2717) (end 110.5 77.79868) (width 0.4) (layer "F.Cu") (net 13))
 (segment (start 122.12132 79.87868) (end 120.61132 79.87868) (width 0.4) (layer "F.Cu") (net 13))
 (via (at 123.57132 82.37868) (size 1.4) (drill 0.85) (layers "F.Cu" "B.Cu") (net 13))
 (via (at 112.24772 79.87868) (size 1.4) (drill 0.85) (layers "F.Cu" "B.Cu") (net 13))
 (segment (start 118.732456 80.37188) (end 112.64992 80.37188) (width 0.4) (layer "B.Cu") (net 13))
 (segment (start 120.739256 82.37868) (end 118.732456 80.37188) (width 0.4) (layer "B.Cu") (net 13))
 (segment (start 112.24772 79.96968) (end 112.24772 79.87868) (width 0.4) (layer "B.Cu") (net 13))
 (segment (start 123.57132 82.37868) (end 120.739256 82.37868) (width 0.4) (layer "B.Cu") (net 13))
 (segment (start 112.24772 79.87868) (end 112.24772 79.49938) (width 0.4) (layer "B.Cu") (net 13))
 (segment (start 112.64992 80.37188) (end 112.24772 79.96968) (width 0.4) (layer "B.Cu") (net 13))
 (segment (start 118.07302 74.67308) (end 120.11742 72.62868) (width 0.4) (layer "F.Cu") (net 3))
 (segment (start 115.62132 78.64868) (end 116.46242 78.64868) (width 0.4) (layer "F.Cu") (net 3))
 (segment (start 116.46242 78.64868) (end 118.07302 77.03808) (width 0.4) (layer "F.Cu") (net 3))
 (segment (start 118.07302 77.03808) (end 118.07302 74.67308) (width 0.4) (layer "F.Cu") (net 3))
 (segment (start 131.83132 72.62868) (end 131.87132 72.58868) (width 0.4) (layer "F.Cu") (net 3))
 (segment (start 120.11742 72.62868) (end 131.83132 72.62868) (width 0.4) (layer "F.Cu") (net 3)))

